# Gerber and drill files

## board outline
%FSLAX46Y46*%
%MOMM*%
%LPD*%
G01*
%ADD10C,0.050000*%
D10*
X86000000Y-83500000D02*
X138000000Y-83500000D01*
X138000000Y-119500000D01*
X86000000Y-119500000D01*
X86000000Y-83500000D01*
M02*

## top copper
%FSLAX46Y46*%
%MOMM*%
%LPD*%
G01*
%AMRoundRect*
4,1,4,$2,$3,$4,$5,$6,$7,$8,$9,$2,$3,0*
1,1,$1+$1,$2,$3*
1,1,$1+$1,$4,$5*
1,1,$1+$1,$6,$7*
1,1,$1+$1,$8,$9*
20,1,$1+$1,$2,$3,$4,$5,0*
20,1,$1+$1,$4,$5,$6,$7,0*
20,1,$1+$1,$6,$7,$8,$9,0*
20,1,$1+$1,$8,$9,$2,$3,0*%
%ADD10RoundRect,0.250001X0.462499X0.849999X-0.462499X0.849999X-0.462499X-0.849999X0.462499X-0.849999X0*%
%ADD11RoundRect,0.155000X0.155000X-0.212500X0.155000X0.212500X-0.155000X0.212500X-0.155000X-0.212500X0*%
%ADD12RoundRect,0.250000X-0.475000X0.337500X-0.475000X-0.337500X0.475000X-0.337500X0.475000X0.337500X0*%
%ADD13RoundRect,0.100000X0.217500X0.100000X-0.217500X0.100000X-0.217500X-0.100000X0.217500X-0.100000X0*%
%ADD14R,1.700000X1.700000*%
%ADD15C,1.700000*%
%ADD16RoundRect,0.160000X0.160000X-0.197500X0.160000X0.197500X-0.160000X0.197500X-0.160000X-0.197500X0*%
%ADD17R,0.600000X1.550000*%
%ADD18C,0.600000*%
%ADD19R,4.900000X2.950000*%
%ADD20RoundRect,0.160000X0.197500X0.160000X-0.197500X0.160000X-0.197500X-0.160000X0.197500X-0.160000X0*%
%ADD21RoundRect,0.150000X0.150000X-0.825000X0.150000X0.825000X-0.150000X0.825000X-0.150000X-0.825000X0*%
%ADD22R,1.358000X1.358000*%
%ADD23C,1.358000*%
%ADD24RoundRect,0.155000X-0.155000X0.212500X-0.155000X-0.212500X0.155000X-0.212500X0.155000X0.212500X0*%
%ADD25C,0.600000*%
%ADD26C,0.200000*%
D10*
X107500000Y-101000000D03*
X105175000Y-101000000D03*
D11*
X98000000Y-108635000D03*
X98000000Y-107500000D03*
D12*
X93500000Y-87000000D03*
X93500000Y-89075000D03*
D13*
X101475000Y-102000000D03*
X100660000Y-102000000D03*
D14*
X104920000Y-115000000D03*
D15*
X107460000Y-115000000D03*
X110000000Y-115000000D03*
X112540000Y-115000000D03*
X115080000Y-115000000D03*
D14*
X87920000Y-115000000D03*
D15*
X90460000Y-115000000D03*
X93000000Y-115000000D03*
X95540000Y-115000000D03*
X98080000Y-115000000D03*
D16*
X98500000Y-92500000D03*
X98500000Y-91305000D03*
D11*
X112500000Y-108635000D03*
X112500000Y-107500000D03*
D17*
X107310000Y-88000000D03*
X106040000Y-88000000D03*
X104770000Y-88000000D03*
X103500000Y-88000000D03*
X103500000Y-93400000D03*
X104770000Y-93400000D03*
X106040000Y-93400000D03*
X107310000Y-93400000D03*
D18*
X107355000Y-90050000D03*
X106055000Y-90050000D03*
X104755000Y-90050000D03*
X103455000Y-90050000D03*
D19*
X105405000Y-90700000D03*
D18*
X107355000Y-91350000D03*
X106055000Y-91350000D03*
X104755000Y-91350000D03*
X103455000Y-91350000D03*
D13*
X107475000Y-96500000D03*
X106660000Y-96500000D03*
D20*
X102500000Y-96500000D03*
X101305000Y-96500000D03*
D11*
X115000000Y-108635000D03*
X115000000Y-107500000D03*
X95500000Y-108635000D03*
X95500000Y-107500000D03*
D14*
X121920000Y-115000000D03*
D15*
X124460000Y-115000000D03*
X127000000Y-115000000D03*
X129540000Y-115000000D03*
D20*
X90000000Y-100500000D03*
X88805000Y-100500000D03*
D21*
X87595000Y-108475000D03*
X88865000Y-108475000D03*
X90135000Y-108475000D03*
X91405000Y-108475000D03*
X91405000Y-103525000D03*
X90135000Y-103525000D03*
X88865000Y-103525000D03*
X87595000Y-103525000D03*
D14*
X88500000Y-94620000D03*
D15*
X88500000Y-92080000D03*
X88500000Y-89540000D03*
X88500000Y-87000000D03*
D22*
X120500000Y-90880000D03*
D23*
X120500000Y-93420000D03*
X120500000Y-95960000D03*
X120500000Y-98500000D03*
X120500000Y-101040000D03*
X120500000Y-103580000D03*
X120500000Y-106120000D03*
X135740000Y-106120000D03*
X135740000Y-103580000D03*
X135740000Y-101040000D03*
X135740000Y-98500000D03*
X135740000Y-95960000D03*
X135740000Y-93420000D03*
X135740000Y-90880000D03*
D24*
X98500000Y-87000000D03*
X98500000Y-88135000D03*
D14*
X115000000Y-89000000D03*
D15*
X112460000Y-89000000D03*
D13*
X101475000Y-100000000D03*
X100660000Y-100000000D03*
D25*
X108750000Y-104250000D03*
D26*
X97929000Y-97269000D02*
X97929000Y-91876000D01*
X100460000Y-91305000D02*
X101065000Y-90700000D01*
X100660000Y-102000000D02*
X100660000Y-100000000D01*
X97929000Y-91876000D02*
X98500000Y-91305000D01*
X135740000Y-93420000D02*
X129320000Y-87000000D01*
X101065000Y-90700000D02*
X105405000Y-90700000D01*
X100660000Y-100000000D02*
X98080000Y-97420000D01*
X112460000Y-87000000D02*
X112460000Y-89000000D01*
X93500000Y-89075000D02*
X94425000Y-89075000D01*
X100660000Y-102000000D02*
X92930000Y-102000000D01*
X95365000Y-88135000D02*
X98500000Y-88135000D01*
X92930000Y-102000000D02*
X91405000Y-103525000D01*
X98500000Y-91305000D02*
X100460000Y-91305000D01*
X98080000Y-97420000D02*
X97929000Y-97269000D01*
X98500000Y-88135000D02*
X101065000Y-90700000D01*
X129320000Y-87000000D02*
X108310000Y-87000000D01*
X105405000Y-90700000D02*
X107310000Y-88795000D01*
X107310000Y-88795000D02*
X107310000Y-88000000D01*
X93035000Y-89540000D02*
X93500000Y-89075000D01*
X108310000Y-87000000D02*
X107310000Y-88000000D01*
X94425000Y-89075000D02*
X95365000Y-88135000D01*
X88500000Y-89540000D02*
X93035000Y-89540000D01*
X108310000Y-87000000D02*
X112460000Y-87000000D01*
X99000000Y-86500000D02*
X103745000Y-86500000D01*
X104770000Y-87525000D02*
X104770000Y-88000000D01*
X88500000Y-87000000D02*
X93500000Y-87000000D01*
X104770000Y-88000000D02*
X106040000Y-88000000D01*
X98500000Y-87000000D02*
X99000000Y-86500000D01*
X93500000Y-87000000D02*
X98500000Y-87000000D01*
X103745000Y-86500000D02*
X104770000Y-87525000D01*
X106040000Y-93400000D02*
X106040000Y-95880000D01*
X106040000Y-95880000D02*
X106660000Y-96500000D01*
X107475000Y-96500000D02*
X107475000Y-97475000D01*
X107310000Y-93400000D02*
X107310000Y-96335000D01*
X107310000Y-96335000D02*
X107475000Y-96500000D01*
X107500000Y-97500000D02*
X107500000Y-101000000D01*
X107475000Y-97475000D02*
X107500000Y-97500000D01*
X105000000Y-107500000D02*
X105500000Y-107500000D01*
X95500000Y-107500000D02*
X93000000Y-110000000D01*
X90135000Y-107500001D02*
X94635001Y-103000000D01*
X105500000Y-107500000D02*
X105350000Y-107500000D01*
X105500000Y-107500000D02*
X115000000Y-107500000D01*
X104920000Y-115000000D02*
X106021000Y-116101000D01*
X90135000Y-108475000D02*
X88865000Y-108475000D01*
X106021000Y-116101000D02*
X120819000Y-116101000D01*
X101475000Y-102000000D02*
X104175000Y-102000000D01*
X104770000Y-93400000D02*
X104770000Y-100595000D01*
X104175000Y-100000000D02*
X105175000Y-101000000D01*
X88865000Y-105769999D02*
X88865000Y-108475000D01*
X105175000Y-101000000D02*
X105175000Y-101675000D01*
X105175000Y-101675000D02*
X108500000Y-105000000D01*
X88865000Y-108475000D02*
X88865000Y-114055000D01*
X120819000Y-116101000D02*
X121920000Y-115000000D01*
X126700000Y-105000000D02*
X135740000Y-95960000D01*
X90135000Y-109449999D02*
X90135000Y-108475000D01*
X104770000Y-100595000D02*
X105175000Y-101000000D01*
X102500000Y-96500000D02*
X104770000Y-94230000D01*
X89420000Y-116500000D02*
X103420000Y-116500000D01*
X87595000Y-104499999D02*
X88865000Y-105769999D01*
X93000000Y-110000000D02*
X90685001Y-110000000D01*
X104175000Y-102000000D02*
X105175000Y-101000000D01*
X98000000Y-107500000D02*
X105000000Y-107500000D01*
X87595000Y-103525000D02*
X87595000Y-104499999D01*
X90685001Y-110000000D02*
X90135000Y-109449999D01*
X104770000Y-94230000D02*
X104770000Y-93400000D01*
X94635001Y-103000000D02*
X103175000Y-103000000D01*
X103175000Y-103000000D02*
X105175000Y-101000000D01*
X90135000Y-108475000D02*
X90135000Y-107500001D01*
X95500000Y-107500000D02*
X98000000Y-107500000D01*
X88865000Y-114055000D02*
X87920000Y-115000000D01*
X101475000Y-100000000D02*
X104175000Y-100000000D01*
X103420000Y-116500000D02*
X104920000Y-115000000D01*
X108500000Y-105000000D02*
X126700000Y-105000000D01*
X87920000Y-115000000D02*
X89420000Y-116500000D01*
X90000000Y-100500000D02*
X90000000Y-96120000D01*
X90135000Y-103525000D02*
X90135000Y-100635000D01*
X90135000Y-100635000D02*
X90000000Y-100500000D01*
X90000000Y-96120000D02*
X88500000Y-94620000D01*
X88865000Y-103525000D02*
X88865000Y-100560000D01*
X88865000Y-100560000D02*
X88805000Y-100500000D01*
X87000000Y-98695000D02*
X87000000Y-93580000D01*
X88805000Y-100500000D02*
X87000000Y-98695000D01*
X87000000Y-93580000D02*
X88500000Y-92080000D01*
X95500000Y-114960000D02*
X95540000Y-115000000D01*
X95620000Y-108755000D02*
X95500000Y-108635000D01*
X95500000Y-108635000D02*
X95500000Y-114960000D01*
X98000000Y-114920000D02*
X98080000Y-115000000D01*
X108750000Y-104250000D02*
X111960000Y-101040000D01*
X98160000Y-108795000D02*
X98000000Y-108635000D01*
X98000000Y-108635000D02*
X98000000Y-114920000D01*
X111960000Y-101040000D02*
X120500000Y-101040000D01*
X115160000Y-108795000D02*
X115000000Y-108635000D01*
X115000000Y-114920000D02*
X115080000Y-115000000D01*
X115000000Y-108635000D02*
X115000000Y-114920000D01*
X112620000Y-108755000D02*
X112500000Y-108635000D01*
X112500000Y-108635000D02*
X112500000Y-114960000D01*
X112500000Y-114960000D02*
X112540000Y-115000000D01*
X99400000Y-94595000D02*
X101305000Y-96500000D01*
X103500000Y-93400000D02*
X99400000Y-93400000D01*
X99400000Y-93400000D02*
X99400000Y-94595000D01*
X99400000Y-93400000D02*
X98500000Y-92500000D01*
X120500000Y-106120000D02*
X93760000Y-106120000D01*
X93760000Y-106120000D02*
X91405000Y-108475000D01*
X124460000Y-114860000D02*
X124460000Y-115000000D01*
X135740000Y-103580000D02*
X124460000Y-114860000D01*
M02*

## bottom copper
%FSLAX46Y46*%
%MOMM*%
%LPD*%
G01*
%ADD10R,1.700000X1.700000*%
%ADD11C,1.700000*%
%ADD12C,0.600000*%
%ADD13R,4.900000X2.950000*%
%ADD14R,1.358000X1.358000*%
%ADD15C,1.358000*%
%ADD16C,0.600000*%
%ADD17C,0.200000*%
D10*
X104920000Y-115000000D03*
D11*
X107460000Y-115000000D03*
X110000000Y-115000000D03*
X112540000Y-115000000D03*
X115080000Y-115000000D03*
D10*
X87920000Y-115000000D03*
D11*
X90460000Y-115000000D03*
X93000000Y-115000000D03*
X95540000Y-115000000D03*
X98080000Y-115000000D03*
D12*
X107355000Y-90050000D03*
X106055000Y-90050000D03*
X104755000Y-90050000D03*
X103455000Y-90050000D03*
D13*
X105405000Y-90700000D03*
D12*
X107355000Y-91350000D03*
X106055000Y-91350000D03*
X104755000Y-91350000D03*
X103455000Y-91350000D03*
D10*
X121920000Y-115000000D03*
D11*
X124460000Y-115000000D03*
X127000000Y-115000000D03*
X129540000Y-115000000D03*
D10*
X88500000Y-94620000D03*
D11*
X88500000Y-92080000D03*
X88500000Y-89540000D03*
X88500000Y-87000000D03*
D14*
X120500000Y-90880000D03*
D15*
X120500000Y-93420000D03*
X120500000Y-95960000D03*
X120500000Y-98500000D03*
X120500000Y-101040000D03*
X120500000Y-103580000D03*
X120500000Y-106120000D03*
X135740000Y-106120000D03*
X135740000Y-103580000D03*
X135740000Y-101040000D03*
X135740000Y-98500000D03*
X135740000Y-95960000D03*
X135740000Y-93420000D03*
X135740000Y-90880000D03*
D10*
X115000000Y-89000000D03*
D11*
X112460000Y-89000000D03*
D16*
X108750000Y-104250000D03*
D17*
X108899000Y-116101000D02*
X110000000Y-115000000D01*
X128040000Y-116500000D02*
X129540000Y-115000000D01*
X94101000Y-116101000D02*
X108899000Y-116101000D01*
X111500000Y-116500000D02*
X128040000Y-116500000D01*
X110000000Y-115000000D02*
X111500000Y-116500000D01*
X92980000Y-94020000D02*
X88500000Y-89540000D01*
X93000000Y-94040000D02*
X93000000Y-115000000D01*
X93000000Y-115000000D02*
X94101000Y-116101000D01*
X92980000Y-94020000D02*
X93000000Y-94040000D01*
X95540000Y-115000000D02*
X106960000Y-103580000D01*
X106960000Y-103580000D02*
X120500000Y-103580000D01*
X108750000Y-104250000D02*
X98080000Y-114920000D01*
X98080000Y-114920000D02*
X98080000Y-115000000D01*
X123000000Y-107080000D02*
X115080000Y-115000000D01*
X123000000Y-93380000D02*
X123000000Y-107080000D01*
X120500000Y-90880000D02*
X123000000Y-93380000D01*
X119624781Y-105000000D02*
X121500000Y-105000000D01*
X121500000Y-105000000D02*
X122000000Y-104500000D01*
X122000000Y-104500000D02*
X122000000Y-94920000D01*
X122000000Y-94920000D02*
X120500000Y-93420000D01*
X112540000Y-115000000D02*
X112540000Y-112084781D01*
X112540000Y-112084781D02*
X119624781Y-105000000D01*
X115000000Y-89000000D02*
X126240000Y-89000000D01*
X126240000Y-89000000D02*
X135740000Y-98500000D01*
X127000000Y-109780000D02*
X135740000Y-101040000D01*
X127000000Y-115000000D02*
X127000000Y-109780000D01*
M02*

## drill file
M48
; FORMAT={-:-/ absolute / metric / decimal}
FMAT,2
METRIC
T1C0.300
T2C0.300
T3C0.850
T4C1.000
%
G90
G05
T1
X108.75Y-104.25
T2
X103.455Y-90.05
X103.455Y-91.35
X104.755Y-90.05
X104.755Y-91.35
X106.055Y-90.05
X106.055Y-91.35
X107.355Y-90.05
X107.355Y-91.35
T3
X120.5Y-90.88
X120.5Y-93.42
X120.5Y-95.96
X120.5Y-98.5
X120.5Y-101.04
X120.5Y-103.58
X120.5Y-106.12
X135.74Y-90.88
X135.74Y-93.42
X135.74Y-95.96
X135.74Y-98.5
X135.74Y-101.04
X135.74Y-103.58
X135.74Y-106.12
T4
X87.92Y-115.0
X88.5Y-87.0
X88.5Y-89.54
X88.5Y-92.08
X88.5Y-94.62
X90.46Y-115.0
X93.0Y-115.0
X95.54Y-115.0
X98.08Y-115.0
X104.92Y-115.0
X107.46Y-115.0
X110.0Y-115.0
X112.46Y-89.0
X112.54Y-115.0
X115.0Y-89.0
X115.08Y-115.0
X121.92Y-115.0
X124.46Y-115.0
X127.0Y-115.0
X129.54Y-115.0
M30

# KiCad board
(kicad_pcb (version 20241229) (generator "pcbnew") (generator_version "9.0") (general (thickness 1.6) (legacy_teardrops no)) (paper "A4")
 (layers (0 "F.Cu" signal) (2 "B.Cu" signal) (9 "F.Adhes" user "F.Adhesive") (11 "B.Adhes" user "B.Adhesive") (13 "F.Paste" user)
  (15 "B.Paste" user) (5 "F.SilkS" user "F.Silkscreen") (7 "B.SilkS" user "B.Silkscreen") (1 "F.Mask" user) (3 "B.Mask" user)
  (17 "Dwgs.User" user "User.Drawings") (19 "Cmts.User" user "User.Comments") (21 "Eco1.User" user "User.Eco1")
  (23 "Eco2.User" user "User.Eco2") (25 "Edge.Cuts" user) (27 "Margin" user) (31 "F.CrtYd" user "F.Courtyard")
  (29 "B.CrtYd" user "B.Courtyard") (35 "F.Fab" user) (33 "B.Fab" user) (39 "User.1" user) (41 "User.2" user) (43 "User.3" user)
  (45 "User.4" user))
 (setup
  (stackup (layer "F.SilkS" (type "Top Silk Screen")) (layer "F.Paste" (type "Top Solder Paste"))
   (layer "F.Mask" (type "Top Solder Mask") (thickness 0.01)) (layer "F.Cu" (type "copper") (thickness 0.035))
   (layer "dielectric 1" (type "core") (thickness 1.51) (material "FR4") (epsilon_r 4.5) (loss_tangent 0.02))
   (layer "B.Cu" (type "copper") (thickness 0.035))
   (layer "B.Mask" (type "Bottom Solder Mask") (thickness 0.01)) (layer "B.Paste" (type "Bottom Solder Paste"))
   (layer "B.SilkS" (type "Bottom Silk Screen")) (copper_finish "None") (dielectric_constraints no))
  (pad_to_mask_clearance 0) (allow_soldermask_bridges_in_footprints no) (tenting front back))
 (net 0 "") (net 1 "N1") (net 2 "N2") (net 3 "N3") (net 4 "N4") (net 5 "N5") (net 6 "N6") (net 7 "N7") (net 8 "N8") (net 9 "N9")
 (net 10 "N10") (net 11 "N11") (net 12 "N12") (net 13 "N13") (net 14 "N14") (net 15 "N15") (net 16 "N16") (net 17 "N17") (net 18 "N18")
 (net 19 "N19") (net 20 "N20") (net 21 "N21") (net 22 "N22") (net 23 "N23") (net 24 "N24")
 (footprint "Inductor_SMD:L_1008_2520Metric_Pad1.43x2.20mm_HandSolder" (layer "F.Cu") (at 106.3375 101 180)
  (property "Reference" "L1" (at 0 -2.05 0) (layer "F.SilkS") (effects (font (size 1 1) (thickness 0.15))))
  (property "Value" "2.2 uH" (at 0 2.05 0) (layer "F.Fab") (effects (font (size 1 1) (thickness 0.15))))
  (pad "1" smd roundrect (at -1.1625 0 180) (size 1.425 2.2) (layers "F.Cu" "F.Mask" "F.Paste") (roundrect_rratio 0.175439) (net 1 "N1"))
  (pad "2" smd roundrect (at 1.1625 0 180) (size 1.425 2.2) (layers "F.Cu" "F.Mask" "F.Paste") (roundrect_rratio 0.175439) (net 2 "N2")))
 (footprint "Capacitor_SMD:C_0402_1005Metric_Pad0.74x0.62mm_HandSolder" (layer "F.Cu") (at 98 108.0675 90)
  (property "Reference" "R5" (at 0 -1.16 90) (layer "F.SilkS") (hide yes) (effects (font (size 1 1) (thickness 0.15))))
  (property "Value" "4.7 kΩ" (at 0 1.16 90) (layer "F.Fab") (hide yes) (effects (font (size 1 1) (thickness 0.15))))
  (pad "1" smd roundrect (at -0.5675 0 90) (size 0.735 0.62) (layers "F.Cu" "F.Mask" "F.Paste") (roundrect_rratio 0.25) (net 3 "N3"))
  (pad "2" smd roundrect (at 0.5675 0 90) (size 0.735 0.62) (layers "F.Cu" "F.Mask" "F.Paste") (roundrect_rratio 0.25) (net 2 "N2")))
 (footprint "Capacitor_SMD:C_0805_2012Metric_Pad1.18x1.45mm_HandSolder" (layer "F.Cu") (at 93.5 88.0375 -90)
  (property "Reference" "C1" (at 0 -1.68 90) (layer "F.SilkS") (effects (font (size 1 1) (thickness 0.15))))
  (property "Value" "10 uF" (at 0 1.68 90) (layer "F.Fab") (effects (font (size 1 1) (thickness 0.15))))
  (pad "1" smd roundrect (at -1.0375 0 270) (size 1.175 1.45) (layers "F.Cu" "F.Mask" "F.Paste") (roundrect_rratio 0.212766) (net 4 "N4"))
  (pad "2" smd roundrect (at 1.0375 0 270) (size 1.175 1.45) (layers "F.Cu" "F.Mask" "F.Paste") (roundrect_rratio 0.212766) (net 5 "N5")))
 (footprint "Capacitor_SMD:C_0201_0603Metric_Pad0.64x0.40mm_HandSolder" (layer "F.Cu") (at 101.0675 102 180)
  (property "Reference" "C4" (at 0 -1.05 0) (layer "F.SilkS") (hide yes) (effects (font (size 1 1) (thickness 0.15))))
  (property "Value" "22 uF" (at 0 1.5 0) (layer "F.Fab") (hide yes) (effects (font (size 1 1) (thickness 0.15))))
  (pad "" smd roundrect (at -0.4325 0 180) (size 0.458 0.36) (layers "F.Paste") (roundrect_rratio 0.25))
  (pad "" smd roundrect (at 0.4325 0 180) (size 0.458 0.36) (layers "F.Paste") (roundrect_rratio 0.25))
  (pad "1" smd roundrect (at -0.4075 0 180) (size 0.635 0.4) (layers "F.Cu" "F.Mask") (roundrect_rratio 0.25) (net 2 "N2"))
  (pad "2" smd roundrect (at 0.4075 0 180) (size 0.635 0.4) (layers "F.Cu" "F.Mask") (roundrect_rratio 0.25) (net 5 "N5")))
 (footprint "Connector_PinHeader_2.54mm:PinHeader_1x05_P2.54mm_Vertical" (layer "F.Cu") (at 104.92 115 90)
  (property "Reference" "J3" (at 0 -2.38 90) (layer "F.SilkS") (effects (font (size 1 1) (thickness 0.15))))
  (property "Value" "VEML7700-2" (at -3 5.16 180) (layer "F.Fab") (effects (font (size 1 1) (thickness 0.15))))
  (pad "1" thru_hole rect (at 0 0 90) (size 1.7 1.7) (drill 1) (layers "*.Cu" "*.Mask") (remove_unused_layers no) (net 2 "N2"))
  (pad "2" thru_hole circle (at 0 2.54 90) (size 1.7 1.7) (drill 1) (layers "*.Cu" "*.Mask") (remove_unused_layers no) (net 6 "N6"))
  (pad "3" thru_hole circle (at 0 5.08 90) (size 1.7 1.7) (drill 1) (layers "*.Cu" "*.Mask") (remove_unused_layers no) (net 5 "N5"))
  (pad "4" thru_hole circle (at 0 7.62 90) (size 1.7 1.7) (drill 1) (layers "*.Cu" "*.Mask") (remove_unused_layers no) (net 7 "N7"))
  (pad "5" thru_hole circle (at 0 10.16 90) (size 1.7 1.7) (drill 1) (layers "*.Cu" "*.Mask") (remove_unused_layers no) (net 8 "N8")))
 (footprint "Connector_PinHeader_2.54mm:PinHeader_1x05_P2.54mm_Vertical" (layer "F.Cu") (at 87.92 115 90)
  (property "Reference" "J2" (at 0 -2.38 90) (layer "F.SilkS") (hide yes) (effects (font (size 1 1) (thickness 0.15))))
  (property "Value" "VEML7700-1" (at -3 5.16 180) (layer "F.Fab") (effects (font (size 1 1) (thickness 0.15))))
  (pad "1" thru_hole rect (at 0 0 90) (size 1.7 1.7) (drill 1) (layers "*.Cu" "*.Mask") (remove_unused_layers no) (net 2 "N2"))
  (pad "2" thru_hole circle (at 0 2.54 90) (size 1.7 1.7) (drill 1) (layers "*.Cu" "*.Mask") (remove_unused_layers no) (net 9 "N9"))
  (pad "3" thru_hole circle (at 0 5.08 90) (size 1.7 1.7) (drill 1) (layers "*.Cu" "*.Mask") (remove_unused_layers no) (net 5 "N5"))
  (pad "4" thru_hole circle (at 0 7.62 90) (size 1.7 1.7) (drill 1) (layers "*.Cu" "*.Mask") (remove_unused_layers no) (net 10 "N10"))
  (pad "5" thru_hole circle (at 0 10.16 90) (size 1.7 1.7) (drill 1) (layers "*.Cu" "*.Mask") (remove_unused_layers no) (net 3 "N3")))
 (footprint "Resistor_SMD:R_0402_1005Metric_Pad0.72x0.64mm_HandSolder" (layer "F.Cu") (at 98.5 91.9025 90)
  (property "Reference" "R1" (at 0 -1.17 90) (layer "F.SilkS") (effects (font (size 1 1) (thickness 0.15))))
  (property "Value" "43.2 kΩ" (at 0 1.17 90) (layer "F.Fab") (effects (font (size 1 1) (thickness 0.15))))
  (pad "1" smd roundrect (at -0.5975 0 90) (size 0.715 0.64) (layers "F.Cu" "F.Mask" "F.Paste") (roundrect_rratio 0.25) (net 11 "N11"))
  (pad "2" smd roundrect (at 0.5975 0 90) (size 0.715 0.64) (layers "F.Cu" "F.Mask" "F.Paste") (roundrect_rratio 0.25) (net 5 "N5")))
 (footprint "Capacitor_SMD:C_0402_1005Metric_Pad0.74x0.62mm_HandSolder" (layer "F.Cu") (at 112.5 108.0675 90)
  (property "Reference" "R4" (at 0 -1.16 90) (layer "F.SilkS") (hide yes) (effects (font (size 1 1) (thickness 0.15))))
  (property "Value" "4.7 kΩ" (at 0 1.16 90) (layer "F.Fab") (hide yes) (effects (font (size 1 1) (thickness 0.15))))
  (pad "1" smd roundrect (at -0.5675 0 90) (size 0.735 0.62) (layers "F.Cu" "F.Mask" "F.Paste") (roundrect_rratio 0.25) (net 7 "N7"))
  (pad "2" smd roundrect (at 0.5675 0 90) (size 0.735 0.62) (layers "F.Cu" "F.Mask" "F.Paste") (roundrect_rratio 0.25) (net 2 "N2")))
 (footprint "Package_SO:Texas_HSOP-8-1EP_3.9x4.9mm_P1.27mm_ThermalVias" (layer "F.Cu") (at 105.405 90.7 -90)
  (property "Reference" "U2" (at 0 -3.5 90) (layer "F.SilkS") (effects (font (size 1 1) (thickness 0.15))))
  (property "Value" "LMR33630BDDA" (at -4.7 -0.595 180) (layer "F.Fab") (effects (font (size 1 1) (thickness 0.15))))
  (pad "" smd rect (at 0 0 270) (size 2.6 3.1) (layers "F.Mask"))
  (pad "" smd rect (at 0 0 270) (size 2.6 3.1) (layers "F.Paste"))
  (pad "1" smd rect (at -2.7 -1.905 270) (size 1.55 0.6) (layers "F.Cu" "F.Mask" "F.Paste") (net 5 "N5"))
  (pad "2" smd rect (at -2.7 -0.635 270) (size 1.55 0.6) (layers "F.Cu" "F.Mask" "F.Paste") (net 4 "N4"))
  (pad "3" smd rect (at -2.7 0.635 270) (size 1.55 0.6) (layers "F.Cu" "F.Mask" "F.Paste") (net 4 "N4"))
  (pad "4" smd rect (at -2.7 1.905 270) (size 1.55 0.6) (layers "F.Cu" "F.Mask" "F.Paste") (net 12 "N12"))
  (pad "5" smd rect (at 2.7 1.905 270) (size 1.55 0.6) (layers "F.Cu" "F.Mask" "F.Paste") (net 11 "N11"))
  (pad "6" smd rect (at 2.7 0.635 270) (size 1.55 0.6) (layers "F.Cu" "F.Mask" "F.Paste") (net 2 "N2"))
  (pad "7" smd rect (at 2.7 -0.635 270) (size 1.55 0.6) (layers "F.Cu" "F.Mask" "F.Paste") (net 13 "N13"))
  (pad "8" smd rect (at 2.7 -1.905 270) (size 1.55 0.6) (layers "F.Cu" "F.Mask" "F.Paste") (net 1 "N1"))
  (pad "9" thru_hole circle (at -0.65 -1.95 270) (size 0.6 0.6) (drill 0.3) (layers "*.Cu") (remove_unused_layers no) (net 5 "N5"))
  (pad "9" thru_hole circle (at -0.65 -0.65 270) (size 0.6 0.6) (drill 0.3) (layers "*.Cu") (remove_unused_layers no) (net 5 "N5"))
  (pad "9" thru_hole circle (at -0.65 0.65 270) (size 0.6 0.6) (drill 0.3) (layers "*.Cu") (remove_unused_layers no) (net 5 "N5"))
  (pad "9" thru_hole circle (at -0.65 1.95 270) (size 0.6 0.6) (drill 0.3) (layers "*.Cu") (remove_unused_layers no) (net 5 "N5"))
  (pad "9" smd rect (at 0 0 270) (size 2.95 4.9) (layers "F.Cu") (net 5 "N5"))
  (pad "9" smd rect (at 0 0 270) (size 2.95 4.9) (layers "B.Cu") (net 5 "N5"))
  (pad "9" thru_hole circle (at 0.65 -1.95 270) (size 0.6 0.6) (drill 0.3) (layers "*.Cu") (remove_unused_layers no) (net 5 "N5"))
  (pad "9" thru_hole circle (at 0.65 -0.65 270) (size 0.6 0.6) (drill 0.3) (layers "*.Cu") (remove_unused_layers no) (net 5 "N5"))
  (pad "9" thru_hole circle (at 0.65 0.65 270) (size 0.6 0.6) (drill 0.3) (layers "*.Cu") (remove_unused_layers no) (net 5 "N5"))
  (pad "9" thru_hole circle (at 0.65 1.95 270) (size 0.6 0.6) (drill 0.3) (layers "*.Cu") (remove_unused_layers no) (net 5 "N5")))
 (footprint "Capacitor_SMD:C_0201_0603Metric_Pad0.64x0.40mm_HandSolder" (layer "F.Cu") (at 107.0675 96.5 180)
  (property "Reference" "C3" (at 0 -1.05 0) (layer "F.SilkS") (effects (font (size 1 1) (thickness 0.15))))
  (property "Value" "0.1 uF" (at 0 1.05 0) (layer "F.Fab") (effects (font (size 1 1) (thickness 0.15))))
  (pad "" smd roundrect (at -0.4325 0 180) (size 0.458 0.36) (layers "F.Paste") (roundrect_rratio 0.25))
  (pad "" smd roundrect (at 0.4325 0 180) (size 0.458 0.36) (layers "F.Paste") (roundrect_rratio 0.25))
  (pad "1" smd roundrect (at -0.4075 0 180) (size 0.635 0.4) (layers "F.Cu" "F.Mask") (roundrect_rratio 0.25) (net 1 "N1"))
  (pad "2" smd roundrect (at 0.4075 0 180) (size 0.635 0.4) (layers "F.Cu" "F.Mask") (roundrect_rratio 0.25) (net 13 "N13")))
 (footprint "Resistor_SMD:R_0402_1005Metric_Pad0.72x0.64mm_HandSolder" (layer "F.Cu") (at 101.9025 96.5 180)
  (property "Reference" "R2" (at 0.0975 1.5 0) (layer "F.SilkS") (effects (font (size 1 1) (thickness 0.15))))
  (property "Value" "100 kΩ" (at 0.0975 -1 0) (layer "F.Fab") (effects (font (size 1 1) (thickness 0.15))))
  (pad "1" smd roundrect (at -0.5975 0 180) (size 0.715 0.64) (layers "F.Cu" "F.Mask" "F.Paste") (roundrect_rratio 0.25) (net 2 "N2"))
  (pad "2" smd roundrect (at 0.5975 0 180) (size 0.715 0.64) (layers "F.Cu" "F.Mask" "F.Paste") (roundrect_rratio 0.25) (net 11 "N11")))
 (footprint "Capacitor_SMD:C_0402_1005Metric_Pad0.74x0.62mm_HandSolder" (layer "F.Cu") (at 115 108.0675 90)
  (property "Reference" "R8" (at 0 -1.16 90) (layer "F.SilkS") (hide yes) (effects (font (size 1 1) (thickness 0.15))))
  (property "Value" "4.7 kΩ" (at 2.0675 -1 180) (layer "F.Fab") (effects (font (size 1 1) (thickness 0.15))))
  (pad "1" smd roundrect (at -0.5675 0 90) (size 0.735 0.62) (layers "F.Cu" "F.Mask" "F.Paste") (roundrect_rratio 0.25) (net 8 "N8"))
  (pad "2" smd roundrect (at 0.5675 0 90) (size 0.735 0.62) (layers "F.Cu" "F.Mask" "F.Paste") (roundrect_rratio 0.25) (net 2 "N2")))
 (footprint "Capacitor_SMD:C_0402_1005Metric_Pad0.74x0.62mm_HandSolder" (layer "F.Cu") (at 95.5 108.0675 90)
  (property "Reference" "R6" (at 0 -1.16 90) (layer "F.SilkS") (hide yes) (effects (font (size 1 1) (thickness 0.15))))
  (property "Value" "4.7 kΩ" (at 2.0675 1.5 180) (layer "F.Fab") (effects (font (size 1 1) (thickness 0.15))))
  (pad "1" smd roundrect (at -0.5675 0 90) (size 0.735 0.62) (layers "F.Cu" "F.Mask" "F.Paste") (roundrect_rratio 0.25) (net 10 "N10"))
  (pad "2" smd roundrect (at 0.5675 0 90) (size 0.735 0.62) (layers "F.Cu" "F.Mask" "F.Paste") (roundrect_rratio 0.25) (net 2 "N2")))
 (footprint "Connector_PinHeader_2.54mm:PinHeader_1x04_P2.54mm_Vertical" (layer "F.Cu") (at 121.92 115 90)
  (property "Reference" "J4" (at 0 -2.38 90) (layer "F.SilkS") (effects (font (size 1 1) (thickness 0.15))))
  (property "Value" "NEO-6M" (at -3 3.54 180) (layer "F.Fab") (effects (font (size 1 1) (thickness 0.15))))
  (pad "1" thru_hole rect (at 0 0 90) (size 1.7 1.7) (drill 1) (layers "*.Cu" "*.Mask") (remove_unused_layers no) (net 2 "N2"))
  (pad "2" thru_hole circle (at 0 2.54 90) (size 1.7 1.7) (drill 1) (layers "*.Cu" "*.Mask") (remove_unused_layers no) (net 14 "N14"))
  (pad "3" thru_hole circle (at 0 5.08 90) (size 1.7 1.7) (drill 1) (layers "*.Cu" "*.Mask") (remove_unused_layers no) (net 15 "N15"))
  (pad "4" thru_hole circle (at 0 7.62 90) (size 1.7 1.7) (drill 1) (layers "*.Cu" "*.Mask") (remove_unused_layers no) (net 5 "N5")))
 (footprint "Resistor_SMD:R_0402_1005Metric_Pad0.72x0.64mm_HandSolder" (layer "F.Cu") (at 89.4025 100.5 180)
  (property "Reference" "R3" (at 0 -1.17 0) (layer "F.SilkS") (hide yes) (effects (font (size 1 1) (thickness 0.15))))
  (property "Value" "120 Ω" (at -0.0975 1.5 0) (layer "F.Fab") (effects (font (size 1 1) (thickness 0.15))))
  (pad "1" smd roundrect (at -0.5975 0 180) (size 0.715 0.64) (layers "F.Cu" "F.Mask" "F.Paste") (roundrect_rratio 0.25) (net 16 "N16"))
  (pad "2" smd roundrect (at 0.5975 0 180) (size 0.715 0.64) (layers "F.Cu" "F.Mask" "F.Paste") (roundrect_rratio 0.25) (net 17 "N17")))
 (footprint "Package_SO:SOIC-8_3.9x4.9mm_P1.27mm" (layer "F.Cu") (at 89.5 106 90)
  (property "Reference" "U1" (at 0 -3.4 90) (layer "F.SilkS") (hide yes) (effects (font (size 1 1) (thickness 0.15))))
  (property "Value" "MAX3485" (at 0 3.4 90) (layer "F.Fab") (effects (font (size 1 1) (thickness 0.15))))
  (pad "1" smd roundrect (at -2.475 -1.905 90) (size 1.95 0.6) (layers "F.Cu" "F.Mask" "F.Paste") (roundrect_rratio 0.25) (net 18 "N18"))
  (pad "2" smd roundrect (at -2.475 -0.635 90) (size 1.95 0.6) (layers "F.Cu" "F.Mask" "F.Paste") (roundrect_rratio 0.25) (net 2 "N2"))
  (pad "3" smd roundrect (at -2.475 0.635 90) (size 1.95 0.6) (layers "F.Cu" "F.Mask" "F.Paste") (roundrect_rratio 0.25) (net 2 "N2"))
  (pad "4" smd roundrect (at -2.475 1.905 90) (size 1.95 0.6) (layers "F.Cu" "F.Mask" "F.Paste") (roundrect_rratio 0.25) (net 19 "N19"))
  (pad "5" smd roundrect (at 2.475 1.905 90) (size 1.95 0.6) (layers "F.Cu" "F.Mask" "F.Paste") (roundrect_rratio 0.25) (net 5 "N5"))
  (pad "6" smd roundrect (at 2.475 0.635 90) (size 1.95 0.6) (layers "F.Cu" "F.Mask" "F.Paste") (roundrect_rratio 0.25) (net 16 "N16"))
  (pad "7" smd roundrect (at 2.475 -0.635 90) (size 1.95 0.6) (layers "F.Cu" "F.Mask" "F.Paste") (roundrect_rratio 0.25) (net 17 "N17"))
  (pad "8" smd roundrect (at 2.475 -1.905 90) (size 1.95 0.6) (layers "F.Cu" "F.Mask" "F.Paste") (roundrect_rratio 0.25) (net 2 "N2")))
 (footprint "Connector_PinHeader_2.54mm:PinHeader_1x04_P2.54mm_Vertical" (layer "F.Cu") (at 88.5 94.62 180)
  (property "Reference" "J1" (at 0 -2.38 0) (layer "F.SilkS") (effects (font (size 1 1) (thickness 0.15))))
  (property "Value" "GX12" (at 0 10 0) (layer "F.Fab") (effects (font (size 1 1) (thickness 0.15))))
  (pad "1" thru_hole rect (at 0 0 180) (size 1.7 1.7) (drill 1) (layers "*.Cu" "*.Mask") (remove_unused_layers no) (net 16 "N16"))
  (pad "2" thru_hole circle (at 0 2.54 180) (size 1.7 1.7) (drill 1) (layers "*.Cu" "*.Mask") (remove_unused_layers no) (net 17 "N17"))
  (pad "3" thru_hole circle (at 0 5.08 180) (size 1.7 1.7) (drill 1) (layers "*.Cu" "*.Mask") (remove_unused_layers no) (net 5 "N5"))
  (pad "4" thru_hole circle (at 0 7.62 180) (size 1.7 1.7) (drill 1) (layers "*.Cu" "*.Mask") (remove_unused_layers no) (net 4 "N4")))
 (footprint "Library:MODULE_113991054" (layer "F.Cu") (at 128.12 98.4365)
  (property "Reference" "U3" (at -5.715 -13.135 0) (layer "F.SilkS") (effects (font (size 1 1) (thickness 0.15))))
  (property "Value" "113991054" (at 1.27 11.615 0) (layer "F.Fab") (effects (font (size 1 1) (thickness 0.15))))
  (pad "1" thru_hole rect (at -7.62 -7.5565) (size 1.358 1.358) (drill 0.85) (layers "*.Cu" "*.Mask") (remove_unused_layers no) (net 8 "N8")
   (solder_mask_margin 0.102))
  (pad "2" thru_hole circle (at -7.62 -5.0165) (size 1.358 1.358) (drill 0.85) (layers "*.Cu" "*.Mask") (remove_unused_layers no)
   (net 7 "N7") (solder_mask_margin 0.102))
  (pad "3" thru_hole circle (at -7.62 -2.4765) (size 1.358 1.358) (drill 0.85) (layers "*.Cu" "*.Mask") (remove_unused_layers no)
   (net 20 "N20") (solder_mask_margin 0.102))
  (pad "4" thru_hole circle (at -7.62 0.0635) (size 1.358 1.358) (drill 0.85) (layers "*.Cu" "*.Mask") (remove_unused_layers no)
   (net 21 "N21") (solder_mask_margin 0.102))
  (pad "5" thru_hole circle (at -7.62 2.6035) (size 1.358 1.358) (drill 0.85) (layers "*.Cu" "*.Mask") (remove_unused_layers no)
   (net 3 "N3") (solder_mask_margin 0.102))
  (pad "6" thru_hole circle (at -7.62 5.1435) (size 1.358 1.358) (drill 0.85) (layers "*.Cu" "*.Mask") (remove_unused_layers no)
   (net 10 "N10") (solder_mask_margin 0.102))
  (pad "7" thru_hole circle (at -7.62 7.6835) (size 1.358 1.358) (drill 0.85) (layers "*.Cu" "*.Mask") (remove_unused_layers no)
   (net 19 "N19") (solder_mask_margin 0.102))
  (pad "8" thru_hole circle (at 7.62 7.6835) (size 1.358 1.358) (drill 0.85) (layers "*.Cu" "*.Mask") (remove_unused_layers no)
   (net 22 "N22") (solder_mask_margin 0.102))
  (pad "9" thru_hole circle (at 7.62 5.1435) (size 1.358 1.358) (drill 0.85) (layers "*.Cu" "*.Mask") (remove_unused_layers no)
   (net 14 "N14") (solder_mask_margin 0.102))
  (pad "10" thru_hole circle (at 7.62 2.6035) (size 1.358 1.358) (drill 0.85) (layers "*.Cu" "*.Mask") (remove_unused_layers no)
   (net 15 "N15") (solder_mask_margin 0.102))
  (pad "11" thru_hole circle (at 7.62 0.0635) (size 1.358 1.358) (drill 0.85) (layers "*.Cu" "*.Mask") (remove_unused_layers no)
   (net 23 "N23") (solder_mask_margin 0.102))
  (pad "12" thru_hole circle (at 7.62 -2.4765) (size 1.358 1.358) (drill 0.85) (layers "*.Cu" "*.Mask") (remove_unused_layers no)
   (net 2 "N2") (solder_mask_margin 0.102))
  (pad "13" thru_hole circle (at 7.62 -5.0165) (size 1.358 1.358) (drill 0.85) (layers "*.Cu" "*.Mask") (remove_unused_layers no)
   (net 5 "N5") (solder_mask_margin 0.102))
  (pad "14" thru_hole circle (at 7.62 -7.5565) (size 1.358 1.358) (drill 0.85) (layers "*.Cu" "*.Mask") (remove_unused_layers no)
   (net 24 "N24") (solder_mask_margin 0.102)))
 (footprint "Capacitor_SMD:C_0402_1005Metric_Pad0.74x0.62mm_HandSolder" (layer "F.Cu") (at 98.5 87.5675 -90)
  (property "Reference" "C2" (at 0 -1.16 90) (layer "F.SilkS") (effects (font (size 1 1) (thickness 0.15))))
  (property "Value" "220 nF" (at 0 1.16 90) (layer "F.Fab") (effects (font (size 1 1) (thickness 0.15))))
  (pad "1" smd roundrect (at -0.5675 0 270) (size 0.735 0.62) (layers "F.Cu" "F.Mask" "F.Paste") (roundrect_rratio 0.25) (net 4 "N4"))
  (pad "2" smd roundrect (at 0.5675 0 270) (size 0.735 0.62) (layers "F.Cu" "F.Mask" "F.Paste") (roundrect_rratio 0.25) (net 5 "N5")))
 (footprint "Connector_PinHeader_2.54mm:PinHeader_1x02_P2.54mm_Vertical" (layer "F.Cu") (at 115 89 -90)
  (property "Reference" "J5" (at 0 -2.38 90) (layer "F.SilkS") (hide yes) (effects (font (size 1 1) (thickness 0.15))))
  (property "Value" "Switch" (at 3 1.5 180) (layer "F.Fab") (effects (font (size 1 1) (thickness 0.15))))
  (pad "1" thru_hole rect (at 0 0 270) (size 1.7 1.7) (drill 1) (layers "*.Cu" "*.Mask") (remove_unused_layers no) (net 23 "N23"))
  (pad "2" thru_hole circle (at 0 2.54 270) (size 1.7 1.7) (drill 1) (layers "*.Cu" "*.Mask") (remove_unused_layers no) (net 5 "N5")))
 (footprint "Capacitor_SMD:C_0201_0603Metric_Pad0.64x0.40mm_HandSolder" (layer "F.Cu") (at 101.0675 100 180)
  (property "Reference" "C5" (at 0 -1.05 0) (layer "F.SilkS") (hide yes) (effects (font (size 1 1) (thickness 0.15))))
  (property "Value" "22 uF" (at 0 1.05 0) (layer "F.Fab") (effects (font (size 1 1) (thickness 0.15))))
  (pad "" smd roundrect (at -0.4325 0 180) (size 0.458 0.36) (layers "F.Paste") (roundrect_rratio 0.25))
  (pad "" smd roundrect (at 0.4325 0 180) (size 0.458 0.36) (layers "F.Paste") (roundrect_rratio 0.25))
  (pad "1" smd roundrect (at -0.4075 0 180) (size 0.635 0.4) (layers "F.Cu" "F.Mask") (roundrect_rratio 0.25) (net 2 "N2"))
  (pad "2" smd roundrect (at 0.4075 0 180) (size 0.635 0.4) (layers "F.Cu" "F.Mask") (roundrect_rratio 0.25) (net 5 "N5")))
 (gr_rect (start 86 83.5) (end 138 119.5) (stroke (width 0.05) (type default)) (fill no) (layer "Edge.Cuts"))
 (segment (start 97.929 97.269) (end 97.929 91.876) (width 0.2) (layer "F.Cu") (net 5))
 (segment (start 100.46 91.305) (end 101.065 90.7) (width 0.2) (layer "F.Cu") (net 5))
 (segment (start 100.66 102) (end 100.66 100) (width 0.2) (layer "F.Cu") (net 5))
 (segment (start 97.929 91.876) (end 98.5 91.305) (width 0.2) (layer "F.Cu") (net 5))
 (segment (start 135.74 93.42) (end 129.32 87) (width 0.2) (layer "F.Cu") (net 5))
 (segment (start 101.065 90.7) (end 105.405 90.7) (width 0.2) (layer "F.Cu") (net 5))
 (segment (start 100.66 100) (end 98.08 97.42) (width 0.2) (layer "F.Cu") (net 5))
 (segment (start 112.46 87) (end 112.46 89) (width 0.2) (layer "F.Cu") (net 5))
 (segment (start 93.5 89.075) (end 94.425 89.075) (width 0.2) (layer "F.Cu") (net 5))
 (segment (start 100.66 102) (end 92.93 102) (width 0.2) (layer "F.Cu") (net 5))
 (segment (start 95.365 88.135) (end 98.5 88.135) (width 0.2) (layer "F.Cu") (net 5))
 (segment (start 92.93 102) (end 91.405 103.525) (width 0.2) (layer "F.Cu") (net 5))
 (segment (start 98.5 91.305) (end 100.46 91.305) (width 0.2) (layer "F.Cu") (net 5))
 (segment (start 98.08 97.42) (end 97.929 97.269) (width 0.2) (layer "F.Cu") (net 5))
 (segment (start 98.5 88.135) (end 101.065 90.7) (width 0.2) (layer "F.Cu") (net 5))
 (segment (start 129.32 87) (end 108.31 87) (width 0.2) (layer "F.Cu") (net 5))
 (segment (start 105.405 90.7) (end 107.31 88.795) (width 0.2) (layer "F.Cu") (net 5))
 (segment (start 107.31 88.795) (end 107.31 88) (width 0.2) (layer "F.Cu") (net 5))
 (segment (start 93.035 89.54) (end 93.5 89.075) (width 0.2) (layer "F.Cu") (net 5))
 (segment (start 108.31 87) (end 107.31 88) (width 0.2) (layer "F.Cu") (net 5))
 (segment (start 94.425 89.075) (end 95.365 88.135) (width 0.2) (layer "F.Cu") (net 5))
 (segment (start 88.5 89.54) (end 93.035 89.54) (width 0.2) (layer "F.Cu") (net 5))
 (segment (start 108.31 87) (end 112.46 87) (width 0.2) (layer "F.Cu") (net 5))
 (segment (start 108.899 116.101) (end 110 115) (width 0.2) (layer "B.Cu") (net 5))
 (segment (start 128.04 116.5) (end 129.54 115) (width 0.2) (layer "B.Cu") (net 5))
 (segment (start 94.101 116.101) (end 108.899 116.101) (width 0.2) (layer "B.Cu") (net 5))
 (segment (start 111.5 116.5) (end 128.04 116.5) (width 0.2) (layer "B.Cu") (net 5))
 (segment (start 110 115) (end 111.5 116.5) (width 0.2) (layer "B.Cu") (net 5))
 (segment (start 92.98 94.02) (end 88.5 89.54) (width 0.2) (layer "B.Cu") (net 5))
 (segment (start 93 94.04) (end 93 115) (width 0.2) (layer "B.Cu") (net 5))
 (segment (start 93 115) (end 94.101 116.101) (width 0.2) (layer "B.Cu") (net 5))
 (segment (start 92.98 94.02) (end 93 94.04) (width 0.2) (layer "B.Cu") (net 5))
 (segment (start 99 86.5) (end 103.745 86.5) (width 0.2) (layer "F.Cu") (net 4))
 (segment (start 104.77 87.525) (end 104.77 88) (width 0.2) (layer "F.Cu") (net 4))
 (segment (start 88.5 87) (end 93.5 87) (width 0.2) (layer "F.Cu") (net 4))
 (segment (start 104.77 88) (end 106.04 88) (width 0.2) (layer "F.Cu") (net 4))
 (segment (start 98.5 87) (end 99 86.5) (width 0.2) (layer "F.Cu") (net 4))
 (segment (start 93.5 87) (end 98.5 87) (width 0.2) (layer "F.Cu") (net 4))
 (segment (start 103.745 86.5) (end 104.77 87.525) (width 0.2) (layer "F.Cu") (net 4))
 (segment (start 106.04 93.4) (end 106.04 95.88) (width 0.2) (layer "F.Cu") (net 13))
 (segment (start 106.04 95.88) (end 106.66 96.5) (width 0.2) (layer "F.Cu") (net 13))
 (segment (start 107.475 96.5) (end 107.475 97.475) (width 0.2) (layer "F.Cu") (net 1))
 (segment (start 107.31 93.4) (end 107.31 96.335) (width 0.2) (layer "F.Cu") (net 1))
 (segment (start 107.31 96.335) (end 107.475 96.5) (width 0.2) (layer "F.Cu") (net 1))
 (segment (start 107.5 97.5) (end 107.5 101) (width 0.2) (layer "F.Cu") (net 1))
 (segment (start 107.475 97.475) (end 107.5 97.5) (width 0.2) (layer "F.Cu") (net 1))
 (segment (start 105 107.5) (end 105.5 107.5) (width 0.2) (layer "F.Cu") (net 2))
 (segment (start 95.5 107.5) (end 93 110) (width 0.2) (layer "F.Cu") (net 2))
 (segment (start 90.135 107.500001) (end 94.635001 103) (width 0.2) (layer "F.Cu") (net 2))
 (segment (start 105.5 107.5) (end 105.35 107.5) (width 0.2) (layer "F.Cu") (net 2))
 (segment (start 105.5 107.5) (end 115 107.5) (width 0.2) (layer "F.Cu") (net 2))
 (segment (start 104.92 115) (end 106.021 116.101) (width 0.2) (layer "F.Cu") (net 2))
 (segment (start 90.135 108.475) (end 88.865 108.475) (width 0.2) (layer "F.Cu") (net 2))
 (segment (start 106.021 116.101) (end 120.819 116.101) (width 0.2) (layer "F.Cu") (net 2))
 (segment (start 101.475 102) (end 104.175 102) (width 0.2) (layer "F.Cu") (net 2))
 (segment (start 104.77 93.4) (end 104.77 100.595) (width 0.2) (layer "F.Cu") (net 2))
 (segment (start 104.175 100) (end 105.175 101) (width 0.2) (layer "F.Cu") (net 2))
 (segment (start 88.865 105.769999) (end 88.865 108.475) (width 0.2) (layer "F.Cu") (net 2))
 (segment (start 105.175 101) (end 105.175 101.675) (width 0.2) (layer "F.Cu") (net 2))
 (segment (start 105.175 101.675) (end 108.5 105) (width 0.2) (layer "F.Cu") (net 2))
 (segment (start 88.865 108.475) (end 88.865 114.055) (width 0.2) (layer "F.Cu") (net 2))
 (segment (start 120.819 116.101) (end 121.92 115) (width 0.2) (layer "F.Cu") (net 2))
 (segment (start 126.7 105) (end 135.74 95.96) (width 0.2) (layer "F.Cu") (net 2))
 (segment (start 90.135 109.449999) (end 90.135 108.475) (width 0.2) (layer "F.Cu") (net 2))
 (segment (start 104.77 100.595) (end 105.175 101) (width 0.2) (layer "F.Cu") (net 2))
 (segment (start 102.5 96.5) (end 104.77 94.23) (width 0.2) (layer "F.Cu") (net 2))
 (segment (start 89.42 116.5) (end 103.42 116.5) (width 0.2) (layer "F.Cu") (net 2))
 (segment (start 87.595 104.499999) (end 88.865 105.769999) (width 0.2) (layer "F.Cu") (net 2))
 (segment (start 93 110) (end 90.685001 110) (width 0.2) (layer "F.Cu") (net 2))
 (segment (start 104.175 102) (end 105.175 101) (width 0.2) (layer "F.Cu") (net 2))
 (segment (start 98 107.5) (end 105 107.5) (width 0.2) (layer "F.Cu") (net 2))
 (segment (start 87.595 103.525) (end 87.595 104.499999) (width 0.2) (layer "F.Cu") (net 2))
 (segment (start 90.685001 110) (end 90.135 109.449999) (width 0.2) (layer "F.Cu") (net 2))
 (segment (start 104.77 94.23) (end 104.77 93.4) (width 0.2) (layer "F.Cu") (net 2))
 (segment (start 94.635001 103) (end 103.175 103) (width 0.2) (layer "F.Cu") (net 2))
 (segment (start 103.175 103) (end 105.175 101) (width 0.2) (layer "F.Cu") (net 2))
 (segment (start 90.135 108.475) (end 90.135 107.500001) (width 0.2) (layer "F.Cu") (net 2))
 (segment (start 95.5 107.5) (end 98 107.5) (width 0.2) (layer "F.Cu") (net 2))
 (segment (start 88.865 114.055) (end 87.92 115) (width 0.2) (layer "F.Cu") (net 2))
 (segment (start 101.475 100) (end 104.175 100) (width 0.2) (layer "F.Cu") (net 2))
 (segment (start 103.42 116.5) (end 104.92 115) (width 0.2) (layer "F.Cu") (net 2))
 (segment (start 108.5 105) (end 126.7 105) (width 0.2) (layer "F.Cu") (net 2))
 (segment (start 87.92 115) (end 89.42 116.5) (width 0.2) (layer "F.Cu") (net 2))
 (segment (start 90 100.5) (end 90 96.12) (width 0.2) (layer "F.Cu") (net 16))
 (segment (start 90.135 103.525) (end 90.135 100.635) (width 0.2) (layer "F.Cu") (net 16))
 (segment (start 90.135 100.635) (end 90 100.5) (width 0.2) (layer "F.Cu") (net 16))
 (segment (start 90 96.12) (end 88.5 94.62) (width 0.2) (layer "F.Cu") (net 16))
 (segment (start 88.865 103.525) (end 88.865 100.56) (width 0.2) (layer "F.Cu") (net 17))
 (segment (start 88.865 100.56) (end 88.805 100.5) (width 0.2) (layer "F.Cu") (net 17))
 (segment (start 87 98.695) (end 87 93.58) (width 0.2) (layer "F.Cu") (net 17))
 (segment (start 88.805 100.5) (end 87 98.695) (width 0.2) (layer "F.Cu") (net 17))
 (segment (start 87 93.58) (end 88.5 92.08) (width 0.2) (layer "F.Cu") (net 17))
 (segment (start 95.5 114.96) (end 95.54 115) (width 0.2) (layer "F.Cu") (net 10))
 (segment (start 95.62 108.755) (end 95.5 108.635) (width 0.2) (layer "F.Cu") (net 10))
 (segment (start 95.5 108.635) (end 95.5 114.96) (width 0.2) (layer "F.Cu") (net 10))
 (segment (start 95.54 115) (end 106.96 103.58) (width 0.2) (layer "B.Cu") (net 10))
 (segment (start 106.96 103.58) (end 120.5 103.58) (width 0.2) (layer "B.Cu") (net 10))
 (segment (start 98 114.92) (end 98.08 115) (width 0.2) (layer "F.Cu") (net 3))
 (segment (start 108.75 104.25) (end 111.96 101.04) (width 0.2) (layer "F.Cu") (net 3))
 (segment (start 98.16 108.795) (end 98 108.635) (width 0.2) (layer "F.Cu") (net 3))
 (segment (start 98 108.635) (end 98 114.92) (width 0.2) (layer "F.Cu") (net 3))
 (segment (start 111.96 101.04) (end 120.5 101.04) (width 0.2) (layer "F.Cu") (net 3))
 (via (at 108.75 104.25) (size 0.6) (drill 0.3) (layers "F.Cu" "B.Cu") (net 3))
 (segment (start 108.75 104.25) (end 98.08 114.92) (width 0.2) (layer "B.Cu") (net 3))
 (segment (start 98.08 114.92) (end 98.08 115) (width 0.2) (layer "B.Cu") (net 3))
 (segment (start 115.16 108.795) (end 115 108.635) (width 0.2) (layer "F.Cu") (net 8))
 (segment (start 115 114.92) (end 115.08 115) (width 0.2) (layer "F.Cu") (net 8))
 (segment (start 115 108.635) (end 115 114.92) (width 0.2) (layer "F.Cu") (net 8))
 (segment (start 123 107.08) (end 115.08 115) (width 0.2) (layer "B.Cu") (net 8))
 (segment (start 123 93.38) (end 123 107.08) (width 0.2) (layer "B.Cu") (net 8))
 (segment (start 120.5 90.88) (end 123 93.38) (width 0.2) (layer "B.Cu") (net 8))
 (segment (start 112.62 108.755) (end 112.5 108.635) (width 0.2) (layer "F.Cu") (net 7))
 (segment (start 112.5 108.635) (end 112.5 114.96) (width 0.2) (layer "F.Cu") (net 7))
 (segment (start 112.5 114.96) (end 112.54 115) (width 0.2) (layer "F.Cu") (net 7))
 (segment (start 119.624781 105) (end 121.5 105) (width 0.2) (layer "B.Cu") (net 7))
 (segment (start 121.5 105) (end 122 104.5) (width 0.2) (layer "B.Cu") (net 7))
 (segment (start 122 104.5) (end 122 94.92) (width 0.2) (layer "B.Cu") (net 7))
 (segment (start 122 94.92) (end 120.5 93.42) (width 0.2) (layer "B.Cu") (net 7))
 (segment (start 112.54 115) (end 112.54 112.084781) (width 0.2) (layer "B.Cu") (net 7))
 (segment (start 112.54 112.084781) (end 119.624781 105) (width 0.2) (layer "B.Cu") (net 7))
 (segment (start 99.4 94.595) (end 101.305 96.5) (width 0.2) (layer "F.Cu") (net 11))
 (segment (start 103.5 93.4) (end 99.4 93.4) (width 0.2) (layer "F.Cu") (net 11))
 (segment (start 99.4 93.4) (end 99.4 94.595) (width 0.2) (layer "F.Cu") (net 11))
 (segment (start 99.4 93.4) (end 98.5 92.5) (width 0.2) (layer "F.Cu") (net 11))
 (segment (start 120.5 106.12) (end 93.76 106.12) (width 0.2) (layer "F.Cu") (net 19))
 (segment (start 93.76 106.12) (end 91.405 108.475) (width 0.2) (layer "F.Cu") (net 19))
 (segment (start 124.46 114.86) (end 124.46 115) (width 0.2) (layer "F.Cu") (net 14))
 (segment (start 135.74 103.58) (end 124.46 114.86) (width 0.2) (layer "F.Cu") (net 14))
 (segment (start 115 89) (end 126.24 89) (width 0.2) (layer "B.Cu") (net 23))
 (segment (start 126.24 89) (end 135.74 98.5) (width 0.2) (layer "B.Cu") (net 23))
 (segment (start 127 109.78) (end 135.74 101.04) (width 0.2) (layer "B.Cu") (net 15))
 (segment (start 127 115) (end 127 109.78) (width 0.2) (layer "B.Cu") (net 15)))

